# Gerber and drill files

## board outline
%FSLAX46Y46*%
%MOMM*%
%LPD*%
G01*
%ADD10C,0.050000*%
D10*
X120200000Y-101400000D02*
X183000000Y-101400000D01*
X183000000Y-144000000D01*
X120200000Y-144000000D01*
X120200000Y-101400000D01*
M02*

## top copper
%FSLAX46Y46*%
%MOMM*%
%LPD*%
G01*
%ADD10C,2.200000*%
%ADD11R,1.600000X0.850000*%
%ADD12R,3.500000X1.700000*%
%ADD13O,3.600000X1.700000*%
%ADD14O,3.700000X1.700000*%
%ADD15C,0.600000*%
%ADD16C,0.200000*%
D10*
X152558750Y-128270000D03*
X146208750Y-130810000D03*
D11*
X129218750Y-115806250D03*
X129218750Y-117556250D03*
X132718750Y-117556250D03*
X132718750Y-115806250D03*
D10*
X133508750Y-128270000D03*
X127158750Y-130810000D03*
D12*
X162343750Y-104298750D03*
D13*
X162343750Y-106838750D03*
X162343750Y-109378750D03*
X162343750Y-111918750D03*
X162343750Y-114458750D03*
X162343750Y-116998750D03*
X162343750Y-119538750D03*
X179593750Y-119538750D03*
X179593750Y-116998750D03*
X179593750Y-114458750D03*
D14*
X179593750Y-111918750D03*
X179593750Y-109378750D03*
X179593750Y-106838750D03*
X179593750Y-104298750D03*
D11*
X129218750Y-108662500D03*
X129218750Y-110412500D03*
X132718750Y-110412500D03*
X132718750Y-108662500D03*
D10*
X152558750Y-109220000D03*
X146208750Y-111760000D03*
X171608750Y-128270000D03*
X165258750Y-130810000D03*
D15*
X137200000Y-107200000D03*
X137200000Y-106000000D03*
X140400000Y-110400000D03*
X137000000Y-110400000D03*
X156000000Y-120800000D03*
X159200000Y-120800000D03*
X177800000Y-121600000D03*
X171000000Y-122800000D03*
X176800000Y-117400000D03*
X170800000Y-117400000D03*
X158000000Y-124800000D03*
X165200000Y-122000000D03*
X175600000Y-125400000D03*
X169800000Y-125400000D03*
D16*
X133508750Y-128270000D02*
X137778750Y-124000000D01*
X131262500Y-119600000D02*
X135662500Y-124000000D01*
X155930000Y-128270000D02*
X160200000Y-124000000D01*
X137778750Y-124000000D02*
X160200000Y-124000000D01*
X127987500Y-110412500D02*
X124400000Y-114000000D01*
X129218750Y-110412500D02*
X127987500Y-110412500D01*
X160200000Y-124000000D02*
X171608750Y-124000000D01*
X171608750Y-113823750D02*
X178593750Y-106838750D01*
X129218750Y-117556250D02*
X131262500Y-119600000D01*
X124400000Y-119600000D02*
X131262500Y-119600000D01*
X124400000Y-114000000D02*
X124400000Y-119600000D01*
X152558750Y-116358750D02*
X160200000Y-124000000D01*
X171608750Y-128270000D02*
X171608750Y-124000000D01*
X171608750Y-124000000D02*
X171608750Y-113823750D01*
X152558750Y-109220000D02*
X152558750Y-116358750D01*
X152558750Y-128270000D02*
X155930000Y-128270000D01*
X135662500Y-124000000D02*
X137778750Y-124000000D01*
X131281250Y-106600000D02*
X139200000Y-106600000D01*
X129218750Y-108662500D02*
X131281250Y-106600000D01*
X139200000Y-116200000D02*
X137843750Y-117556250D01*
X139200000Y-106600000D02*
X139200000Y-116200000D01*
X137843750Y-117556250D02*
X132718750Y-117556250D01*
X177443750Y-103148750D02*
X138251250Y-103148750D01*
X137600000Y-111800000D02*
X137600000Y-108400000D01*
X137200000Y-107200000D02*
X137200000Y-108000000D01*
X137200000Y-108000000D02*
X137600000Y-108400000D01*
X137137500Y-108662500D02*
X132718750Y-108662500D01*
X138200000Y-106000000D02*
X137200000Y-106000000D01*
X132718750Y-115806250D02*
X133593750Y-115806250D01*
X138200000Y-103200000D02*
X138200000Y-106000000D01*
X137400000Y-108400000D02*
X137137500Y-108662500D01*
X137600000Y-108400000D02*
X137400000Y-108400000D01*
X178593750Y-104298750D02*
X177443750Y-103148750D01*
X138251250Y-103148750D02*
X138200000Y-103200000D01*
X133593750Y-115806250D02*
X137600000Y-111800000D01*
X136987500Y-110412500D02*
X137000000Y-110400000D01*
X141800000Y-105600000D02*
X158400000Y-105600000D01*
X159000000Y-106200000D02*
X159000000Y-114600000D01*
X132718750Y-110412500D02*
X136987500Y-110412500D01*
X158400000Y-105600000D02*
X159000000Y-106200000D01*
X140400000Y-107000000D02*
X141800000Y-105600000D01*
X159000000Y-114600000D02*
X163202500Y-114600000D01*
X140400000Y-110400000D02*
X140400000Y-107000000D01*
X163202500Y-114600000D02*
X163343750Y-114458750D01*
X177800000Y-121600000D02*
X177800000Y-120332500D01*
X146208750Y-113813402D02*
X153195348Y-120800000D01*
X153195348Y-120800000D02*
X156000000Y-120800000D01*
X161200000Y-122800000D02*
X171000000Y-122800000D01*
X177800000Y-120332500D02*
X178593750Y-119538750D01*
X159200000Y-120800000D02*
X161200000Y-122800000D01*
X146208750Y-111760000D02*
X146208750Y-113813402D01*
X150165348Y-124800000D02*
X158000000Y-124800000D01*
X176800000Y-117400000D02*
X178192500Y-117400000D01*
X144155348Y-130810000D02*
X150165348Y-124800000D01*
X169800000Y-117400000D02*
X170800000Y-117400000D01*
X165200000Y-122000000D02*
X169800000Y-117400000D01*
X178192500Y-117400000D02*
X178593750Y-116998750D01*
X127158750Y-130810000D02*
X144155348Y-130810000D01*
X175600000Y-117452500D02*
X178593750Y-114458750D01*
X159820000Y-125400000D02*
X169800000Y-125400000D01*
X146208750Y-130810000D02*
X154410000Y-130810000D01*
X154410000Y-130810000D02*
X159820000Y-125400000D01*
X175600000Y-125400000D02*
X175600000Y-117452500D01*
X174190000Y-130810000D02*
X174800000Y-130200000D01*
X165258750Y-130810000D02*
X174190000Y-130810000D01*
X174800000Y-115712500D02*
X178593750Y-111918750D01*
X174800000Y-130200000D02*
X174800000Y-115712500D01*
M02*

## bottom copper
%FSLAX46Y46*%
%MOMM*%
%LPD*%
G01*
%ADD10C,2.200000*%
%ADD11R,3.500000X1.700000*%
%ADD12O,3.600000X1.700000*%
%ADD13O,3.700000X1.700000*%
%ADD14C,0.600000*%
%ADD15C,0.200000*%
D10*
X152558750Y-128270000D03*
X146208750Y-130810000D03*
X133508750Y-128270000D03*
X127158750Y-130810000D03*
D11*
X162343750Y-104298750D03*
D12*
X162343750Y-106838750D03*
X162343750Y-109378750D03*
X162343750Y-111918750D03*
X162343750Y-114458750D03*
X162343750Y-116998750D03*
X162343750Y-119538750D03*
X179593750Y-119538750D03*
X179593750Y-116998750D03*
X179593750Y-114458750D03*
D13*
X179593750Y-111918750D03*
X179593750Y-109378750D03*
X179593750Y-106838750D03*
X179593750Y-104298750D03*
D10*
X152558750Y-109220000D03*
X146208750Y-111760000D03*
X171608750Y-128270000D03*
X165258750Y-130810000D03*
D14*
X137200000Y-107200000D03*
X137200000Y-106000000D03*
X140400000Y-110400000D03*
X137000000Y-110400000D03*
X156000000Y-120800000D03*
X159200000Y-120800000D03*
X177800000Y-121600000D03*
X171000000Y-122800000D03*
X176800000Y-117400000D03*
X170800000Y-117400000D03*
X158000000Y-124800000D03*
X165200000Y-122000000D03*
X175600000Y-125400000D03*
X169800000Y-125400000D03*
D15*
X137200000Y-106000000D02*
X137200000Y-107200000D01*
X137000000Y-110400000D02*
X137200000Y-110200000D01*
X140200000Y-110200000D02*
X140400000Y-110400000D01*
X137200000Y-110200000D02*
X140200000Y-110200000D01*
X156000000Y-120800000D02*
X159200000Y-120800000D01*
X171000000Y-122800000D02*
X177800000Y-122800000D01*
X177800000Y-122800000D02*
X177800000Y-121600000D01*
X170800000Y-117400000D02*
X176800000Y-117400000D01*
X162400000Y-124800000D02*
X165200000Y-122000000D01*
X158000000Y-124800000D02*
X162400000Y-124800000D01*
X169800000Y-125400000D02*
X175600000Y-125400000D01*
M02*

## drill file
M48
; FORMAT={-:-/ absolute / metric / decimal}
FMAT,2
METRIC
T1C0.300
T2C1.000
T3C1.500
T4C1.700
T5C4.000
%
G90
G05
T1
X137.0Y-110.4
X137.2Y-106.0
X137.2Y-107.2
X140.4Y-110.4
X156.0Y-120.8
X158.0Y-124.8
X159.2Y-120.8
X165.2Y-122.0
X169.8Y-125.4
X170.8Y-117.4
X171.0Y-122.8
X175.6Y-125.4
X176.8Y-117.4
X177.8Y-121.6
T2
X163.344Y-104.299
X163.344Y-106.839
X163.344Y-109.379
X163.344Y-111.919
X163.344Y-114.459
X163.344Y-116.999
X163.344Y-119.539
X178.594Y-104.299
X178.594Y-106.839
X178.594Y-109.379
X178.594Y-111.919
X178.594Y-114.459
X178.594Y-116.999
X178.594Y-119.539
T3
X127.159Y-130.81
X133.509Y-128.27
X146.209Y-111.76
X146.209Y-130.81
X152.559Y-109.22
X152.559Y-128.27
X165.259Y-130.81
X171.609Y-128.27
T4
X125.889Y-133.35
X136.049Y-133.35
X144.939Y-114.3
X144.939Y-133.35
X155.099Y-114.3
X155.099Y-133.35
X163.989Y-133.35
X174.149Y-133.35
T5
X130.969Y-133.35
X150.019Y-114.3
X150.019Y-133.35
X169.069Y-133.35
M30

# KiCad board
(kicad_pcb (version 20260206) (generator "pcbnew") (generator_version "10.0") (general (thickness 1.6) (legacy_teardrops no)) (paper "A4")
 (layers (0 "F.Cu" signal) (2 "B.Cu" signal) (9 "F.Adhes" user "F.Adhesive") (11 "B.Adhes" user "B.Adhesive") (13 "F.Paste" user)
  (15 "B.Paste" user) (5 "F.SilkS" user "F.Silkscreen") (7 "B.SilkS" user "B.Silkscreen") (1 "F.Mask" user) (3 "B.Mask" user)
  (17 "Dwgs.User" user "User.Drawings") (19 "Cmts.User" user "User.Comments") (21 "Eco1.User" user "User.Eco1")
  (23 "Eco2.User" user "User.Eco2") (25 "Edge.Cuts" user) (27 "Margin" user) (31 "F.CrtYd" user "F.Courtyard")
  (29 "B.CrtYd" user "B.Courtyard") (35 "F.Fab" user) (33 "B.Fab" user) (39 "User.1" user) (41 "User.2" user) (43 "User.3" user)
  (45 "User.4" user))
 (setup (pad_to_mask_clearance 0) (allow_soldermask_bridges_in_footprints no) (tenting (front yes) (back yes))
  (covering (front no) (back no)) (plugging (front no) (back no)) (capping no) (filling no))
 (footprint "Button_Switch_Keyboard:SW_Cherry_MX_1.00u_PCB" (layer "F.Cu") (at 152.55875 128.27)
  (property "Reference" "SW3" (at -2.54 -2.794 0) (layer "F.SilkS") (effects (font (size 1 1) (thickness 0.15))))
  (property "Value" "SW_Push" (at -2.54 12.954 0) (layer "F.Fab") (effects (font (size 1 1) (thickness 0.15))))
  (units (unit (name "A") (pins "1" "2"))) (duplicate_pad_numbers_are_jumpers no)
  (pad "" np_thru_hole circle (at -7.62 5.08) (size 1.7 1.7) (drill 1.7) (layers "*.Cu" "*.Mask"))
  (pad "" np_thru_hole circle (at -2.54 5.08) (size 4 4) (drill 4) (layers "*.Cu" "*.Mask"))
  (pad "" np_thru_hole circle (at 2.54 5.08) (size 1.7 1.7) (drill 1.7) (layers "*.Cu" "*.Mask"))
  (pad "1" thru_hole circle (at 0 0) (size 2.2 2.2) (drill 1.5) (layers "*.Cu" "*.Mask") (remove_unused_layers no) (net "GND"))
  (pad "2" thru_hole circle (at -6.35 2.54) (size 2.2 2.2) (drill 1.5) (layers "*.Cu" "*.Mask") (remove_unused_layers no)
   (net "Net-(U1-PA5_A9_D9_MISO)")))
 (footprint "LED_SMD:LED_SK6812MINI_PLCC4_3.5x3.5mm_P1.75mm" (layer "F.Cu") (at 130.96875 116.68125)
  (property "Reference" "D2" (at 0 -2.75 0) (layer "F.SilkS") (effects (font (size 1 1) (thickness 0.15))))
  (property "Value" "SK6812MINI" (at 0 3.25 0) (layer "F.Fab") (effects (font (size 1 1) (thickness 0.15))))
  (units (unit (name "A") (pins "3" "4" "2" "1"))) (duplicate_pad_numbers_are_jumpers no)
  (pad "1" smd rect (at -1.75 -0.875) (size 1.6 0.85) (layers "F.Cu" "F.Mask" "F.Paste") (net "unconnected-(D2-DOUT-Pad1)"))
  (pad "2" smd rect (at -1.75 0.875) (size 1.6 0.85) (layers "F.Cu" "F.Mask" "F.Paste") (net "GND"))
  (pad "3" smd rect (at 1.75 0.875) (size 1.6 0.85) (layers "F.Cu" "F.Mask" "F.Paste") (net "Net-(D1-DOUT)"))
  (pad "4" smd rect (at 1.75 -0.875) (size 1.6 0.85) (layers "F.Cu" "F.Mask" "F.Paste") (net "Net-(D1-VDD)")))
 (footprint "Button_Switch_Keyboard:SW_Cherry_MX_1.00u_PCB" (layer "F.Cu") (at 133.50875 128.27)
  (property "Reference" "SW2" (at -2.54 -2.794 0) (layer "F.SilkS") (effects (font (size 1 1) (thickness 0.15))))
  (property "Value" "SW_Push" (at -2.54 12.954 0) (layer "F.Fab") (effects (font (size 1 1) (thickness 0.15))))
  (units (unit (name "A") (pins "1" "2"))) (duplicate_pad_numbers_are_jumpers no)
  (pad "" np_thru_hole circle (at -7.62 5.08) (size 1.7 1.7) (drill 1.7) (layers "*.Cu" "*.Mask"))
  (pad "" np_thru_hole circle (at -2.54 5.08) (size 4 4) (drill 4) (layers "*.Cu" "*.Mask"))
  (pad "" np_thru_hole circle (at 2.54 5.08) (size 1.7 1.7) (drill 1.7) (layers "*.Cu" "*.Mask"))
  (pad "1" thru_hole circle (at 0 0) (size 2.2 2.2) (drill 1.5) (layers "*.Cu" "*.Mask") (remove_unused_layers no) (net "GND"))
  (pad "2" thru_hole circle (at -6.35 2.54) (size 2.2 2.2) (drill 1.5) (layers "*.Cu" "*.Mask") (remove_unused_layers no)
   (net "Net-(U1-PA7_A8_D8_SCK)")))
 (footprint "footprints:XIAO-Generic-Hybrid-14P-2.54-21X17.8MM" (layer "F.Cu") (at 170.96875 111.91875)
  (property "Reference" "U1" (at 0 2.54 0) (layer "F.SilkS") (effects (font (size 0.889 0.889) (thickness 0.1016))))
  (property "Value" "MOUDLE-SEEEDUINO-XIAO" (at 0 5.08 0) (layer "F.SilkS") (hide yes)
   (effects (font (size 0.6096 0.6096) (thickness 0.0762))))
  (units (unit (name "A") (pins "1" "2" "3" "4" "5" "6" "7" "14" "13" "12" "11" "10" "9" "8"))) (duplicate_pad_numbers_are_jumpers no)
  (pad "1" thru_hole rect (at -7.625 -7.62) (size 3.5 1.7) (drill 1 (offset -1 0)) (layers "*.Cu" "*.Mask") (remove_unused_layers no)
   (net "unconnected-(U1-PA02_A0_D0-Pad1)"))
  (pad "2" thru_hole oval (at -7.625 -5.08) (size 3.6 1.7) (drill 1 (offset -1 0)) (layers "*.Cu" "*.Mask") (remove_unused_layers no)
   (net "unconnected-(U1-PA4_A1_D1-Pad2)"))
  (pad "3" thru_hole oval (at -7.625 -2.54) (size 3.6 1.7) (drill 1 (offset -1 0)) (layers "*.Cu" "*.Mask") (remove_unused_layers no)
   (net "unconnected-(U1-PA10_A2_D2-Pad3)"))
  (pad "4" thru_hole oval (at -7.625 0) (size 3.6 1.7) (drill 1 (offset -1 0)) (layers "*.Cu" "*.Mask") (remove_unused_layers no)
   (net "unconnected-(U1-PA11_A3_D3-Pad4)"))
  (pad "5" thru_hole oval (at -7.625 2.54) (size 3.6 1.7) (drill 1 (offset -1 0)) (layers "*.Cu" "*.Mask") (remove_unused_layers no)
   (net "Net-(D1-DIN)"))
  (pad "6" thru_hole oval (at -7.625 5.08 180) (size 3.6 1.7) (drill 1 (offset 1 0)) (layers "*.Cu" "*.Mask") (remove_unused_layers no)
   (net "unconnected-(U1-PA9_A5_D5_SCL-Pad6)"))
  (pad "7" thru_hole oval (at -7.625 7.62) (size 3.6 1.7) (drill 1 (offset -1 0)) (layers "*.Cu" "*.Mask") (remove_unused_layers no)
   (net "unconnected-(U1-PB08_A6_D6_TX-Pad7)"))
  (pad "8" thru_hole oval (at 7.625 7.62) (size 3.6 1.7) (drill 1 (offset 1 0)) (layers "*.Cu" "*.Mask") (remove_unused_layers no)
   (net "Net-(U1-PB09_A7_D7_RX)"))
  (pad "9" thru_hole oval (at 7.625 5.08) (size 3.6 1.7) (drill 1 (offset 1 0)) (layers "*.Cu" "*.Mask") (remove_unused_layers no)
   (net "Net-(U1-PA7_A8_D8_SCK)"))
  (pad "10" thru_hole oval (at 7.625 2.54) (size 3.6 1.7) (drill 1 (offset 1 0)) (layers "*.Cu" "*.Mask") (remove_unused_layers no)
   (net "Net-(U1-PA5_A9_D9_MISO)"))
  (pad "11" thru_hole oval (at 7.625 0) (size 3.7 1.7) (drill 1 (offset 1 0)) (layers "*.Cu" "*.Mask") (remove_unused_layers no)
   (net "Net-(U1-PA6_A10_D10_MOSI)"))
  (pad "12" thru_hole oval (at 7.625 -2.54) (size 3.7 1.7) (drill 1 (offset 1 0)) (layers "*.Cu" "*.Mask") (remove_unused_layers no)
   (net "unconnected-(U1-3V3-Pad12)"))
  (pad "13" thru_hole oval (at 7.625 -5.08) (size 3.7 1.7) (drill 1 (offset 1 0)) (layers "*.Cu" "*.Mask") (remove_unused_layers no)
   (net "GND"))
  (pad "14" thru_hole oval (at 7.625 -7.62) (size 3.7 1.7) (drill 1 (offset 1 0)) (layers "*.Cu" "*.Mask") (remove_unused_layers no)
   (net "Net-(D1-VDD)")))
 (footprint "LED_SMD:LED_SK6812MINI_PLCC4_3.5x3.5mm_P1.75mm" (layer "F.Cu") (at 130.96875 109.5375)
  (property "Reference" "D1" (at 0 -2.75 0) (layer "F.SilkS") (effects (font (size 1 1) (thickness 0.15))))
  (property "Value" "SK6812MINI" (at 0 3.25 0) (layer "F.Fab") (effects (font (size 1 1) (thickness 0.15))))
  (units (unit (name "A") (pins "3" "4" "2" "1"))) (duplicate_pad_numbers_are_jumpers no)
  (pad "1" smd rect (at -1.75 -0.875) (size 1.6 0.85) (layers "F.Cu" "F.Mask" "F.Paste") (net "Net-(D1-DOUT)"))
  (pad "2" smd rect (at -1.75 0.875) (size 1.6 0.85) (layers "F.Cu" "F.Mask" "F.Paste") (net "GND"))
  (pad "3" smd rect (at 1.75 0.875) (size 1.6 0.85) (layers "F.Cu" "F.Mask" "F.Paste") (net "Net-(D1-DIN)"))
  (pad "4" smd rect (at 1.75 -0.875) (size 1.6 0.85) (layers "F.Cu" "F.Mask" "F.Paste") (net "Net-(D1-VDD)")))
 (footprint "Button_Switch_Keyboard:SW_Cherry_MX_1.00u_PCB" (layer "F.Cu") (at 152.55875 109.22)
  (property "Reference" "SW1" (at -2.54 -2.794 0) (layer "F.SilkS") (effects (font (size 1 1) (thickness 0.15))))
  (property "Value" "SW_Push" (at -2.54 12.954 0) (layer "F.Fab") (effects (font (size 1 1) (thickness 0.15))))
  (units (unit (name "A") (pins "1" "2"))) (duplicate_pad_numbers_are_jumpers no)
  (pad "" np_thru_hole circle (at -7.62 5.08) (size 1.7 1.7) (drill 1.7) (layers "*.Cu" "*.Mask"))
  (pad "" np_thru_hole circle (at -2.54 5.08) (size 4 4) (drill 4) (layers "*.Cu" "*.Mask"))
  (pad "" np_thru_hole circle (at 2.54 5.08) (size 1.7 1.7) (drill 1.7) (layers "*.Cu" "*.Mask"))
  (pad "1" thru_hole circle (at 0 0) (size 2.2 2.2) (drill 1.5) (layers "*.Cu" "*.Mask") (remove_unused_layers no) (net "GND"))
  (pad "2" thru_hole circle (at -6.35 2.54) (size 2.2 2.2) (drill 1.5) (layers "*.Cu" "*.Mask") (remove_unused_layers no)
   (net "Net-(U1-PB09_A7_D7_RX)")))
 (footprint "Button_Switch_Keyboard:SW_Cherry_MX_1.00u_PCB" (layer "F.Cu") (at 171.60875 128.27)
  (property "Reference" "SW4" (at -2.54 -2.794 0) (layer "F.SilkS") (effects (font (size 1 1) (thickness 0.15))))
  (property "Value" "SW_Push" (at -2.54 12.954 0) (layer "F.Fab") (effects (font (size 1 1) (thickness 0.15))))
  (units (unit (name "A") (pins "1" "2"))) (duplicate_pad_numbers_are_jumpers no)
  (pad "" np_thru_hole circle (at -7.62 5.08) (size 1.7 1.7) (drill 1.7) (layers "*.Cu" "*.Mask"))
  (pad "" np_thru_hole circle (at -2.54 5.08) (size 4 4) (drill 4) (layers "*.Cu" "*.Mask"))
  (pad "" np_thru_hole circle (at 2.54 5.08) (size 1.7 1.7) (drill 1.7) (layers "*.Cu" "*.Mask"))
  (pad "1" thru_hole circle (at 0 0) (size 2.2 2.2) (drill 1.5) (layers "*.Cu" "*.Mask") (remove_unused_layers no) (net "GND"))
  (pad "2" thru_hole circle (at -6.35 2.54) (size 2.2 2.2) (drill 1.5) (layers "*.Cu" "*.Mask") (remove_unused_layers no)
   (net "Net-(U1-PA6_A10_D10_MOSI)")))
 (gr_rect (start 120.2 101.4) (end 183 144) (stroke (width 0.05) (type default)) (fill no) (layer "Edge.Cuts"))
 (segment (start 133.50875 128.27) (end 137.77875 124) (width 0.2) (layer "F.Cu") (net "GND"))
 (segment (start 131.2625 119.6) (end 135.6625 124) (width 0.2) (layer "F.Cu") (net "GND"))
 (segment (start 155.93 128.27) (end 160.2 124) (width 0.2) (layer "F.Cu") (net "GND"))
 (segment (start 137.77875 124) (end 160.2 124) (width 0.2) (layer "F.Cu") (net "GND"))
 (segment (start 127.9875 110.4125) (end 124.4 114) (width 0.2) (layer "F.Cu") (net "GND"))
 (segment (start 129.21875 110.4125) (end 127.9875 110.4125) (width 0.2) (layer "F.Cu") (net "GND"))
 (segment (start 160.2 124) (end 171.60875 124) (width 0.2) (layer "F.Cu") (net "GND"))
 (segment (start 171.60875 113.82375) (end 178.59375 106.83875) (width 0.2) (layer "F.Cu") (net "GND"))
 (segment (start 129.21875 117.55625) (end 131.2625 119.6) (width 0.2) (layer "F.Cu") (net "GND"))
 (segment (start 124.4 119.6) (end 131.2625 119.6) (width 0.2) (layer "F.Cu") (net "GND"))
 (segment (start 124.4 114) (end 124.4 119.6) (width 0.2) (layer "F.Cu") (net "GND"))
 (segment (start 152.55875 116.35875) (end 160.2 124) (width 0.2) (layer "F.Cu") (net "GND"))
 (segment (start 171.60875 128.27) (end 171.60875 124) (width 0.2) (layer "F.Cu") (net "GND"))
 (segment (start 171.60875 124) (end 171.60875 113.82375) (width 0.2) (layer "F.Cu") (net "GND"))
 (segment (start 152.55875 109.22) (end 152.55875 116.35875) (width 0.2) (layer "F.Cu") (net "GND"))
 (segment (start 152.55875 128.27) (end 155.93 128.27) (width 0.2) (layer "F.Cu") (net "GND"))
 (segment (start 135.6625 124) (end 137.77875 124) (width 0.2) (layer "F.Cu") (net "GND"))
 (segment (start 131.28125 106.6) (end 139.2 106.6) (width 0.2) (layer "F.Cu") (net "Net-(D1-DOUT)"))
 (segment (start 129.21875 108.6625) (end 131.28125 106.6) (width 0.2) (layer "F.Cu") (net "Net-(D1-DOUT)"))
 (segment (start 139.2 116.2) (end 137.84375 117.55625) (width 0.2) (layer "F.Cu") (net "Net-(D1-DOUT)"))
 (segment (start 139.2 106.6) (end 139.2 116.2) (width 0.2) (layer "F.Cu") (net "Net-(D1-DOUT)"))
 (segment (start 137.84375 117.55625) (end 132.71875 117.55625) (width 0.2) (layer "F.Cu") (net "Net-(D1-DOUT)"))
 (segment (start 177.44375 103.14875) (end 138.25125 103.14875) (width 0.2) (layer "F.Cu") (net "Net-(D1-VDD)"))
 (segment (start 137.6 111.8) (end 137.6 108.4) (width 0.2) (layer "F.Cu") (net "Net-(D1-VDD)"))
 (segment (start 137.2 107.2) (end 137.2 108) (width 0.2) (layer "F.Cu") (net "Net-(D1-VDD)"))
 (segment (start 137.2 108) (end 137.6 108.4) (width 0.2) (layer "F.Cu") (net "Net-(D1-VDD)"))
 (segment (start 137.1375 108.6625) (end 132.71875 108.6625) (width 0.2) (layer "F.Cu") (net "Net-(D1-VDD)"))
 (segment (start 138.2 106) (end 137.2 106) (width 0.2) (layer "F.Cu") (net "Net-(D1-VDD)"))
 (segment (start 132.71875 115.80625) (end 133.59375 115.80625) (width 0.2) (layer "F.Cu") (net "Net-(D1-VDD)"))
 (segment (start 138.2 103.2) (end 138.2 106) (width 0.2) (layer "F.Cu") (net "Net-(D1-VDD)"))
 (segment (start 137.4 108.4) (end 137.1375 108.6625) (width 0.2) (layer "F.Cu") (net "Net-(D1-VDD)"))
 (segment (start 137.6 108.4) (end 137.4 108.4) (width 0.2) (layer "F.Cu") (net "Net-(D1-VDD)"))
 (segment (start 178.59375 104.29875) (end 177.44375 103.14875) (width 0.2) (layer "F.Cu") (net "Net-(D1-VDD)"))
 (segment (start 138.25125 103.14875) (end 138.2 103.2) (width 0.2) (layer "F.Cu") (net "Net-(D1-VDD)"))
 (segment (start 133.59375 115.80625) (end 137.6 111.8) (width 0.2) (layer "F.Cu") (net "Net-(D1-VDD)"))
 (via (at 137.2 107.2) (size 0.6) (drill 0.3) (layers "F.Cu" "B.Cu") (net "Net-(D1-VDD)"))
 (via (at 137.2 106) (size 0.6) (drill 0.3) (layers "F.Cu" "B.Cu") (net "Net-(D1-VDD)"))
 (segment (start 137.2 106) (end 137.2 107.2) (width 0.2) (layer "B.Cu") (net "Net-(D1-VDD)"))
 (segment (start 136.9875 110.4125) (end 137 110.4) (width 0.2) (layer "F.Cu") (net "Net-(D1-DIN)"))
 (segment (start 141.8 105.6) (end 158.4 105.6) (width 0.2) (layer "F.Cu") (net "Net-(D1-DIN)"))
 (segment (start 159 106.2) (end 159 114.6) (width 0.2) (layer "F.Cu") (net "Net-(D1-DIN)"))
 (segment (start 132.71875 110.4125) (end 136.9875 110.4125) (width 0.2) (layer "F.Cu") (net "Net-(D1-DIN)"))
 (segment (start 158.4 105.6) (end 159 106.2) (width 0.2) (layer "F.Cu") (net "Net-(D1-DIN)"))
 (segment (start 140.4 107) (end 141.8 105.6) (width 0.2) (layer "F.Cu") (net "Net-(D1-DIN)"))
 (segment (start 159 114.6) (end 163.2025 114.6) (width 0.2) (layer "F.Cu") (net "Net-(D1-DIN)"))
 (segment (start 140.4 110.4) (end 140.4 107) (width 0.2) (layer "F.Cu") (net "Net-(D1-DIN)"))
 (segment (start 163.2025 114.6) (end 163.34375 114.45875) (width 0.2) (layer "F.Cu") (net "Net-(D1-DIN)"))
 (via (at 140.4 110.4) (size 0.6) (drill 0.3) (layers "F.Cu" "B.Cu") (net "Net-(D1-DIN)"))
 (via (at 137 110.4) (size 0.6) (drill 0.3) (layers "F.Cu" "B.Cu") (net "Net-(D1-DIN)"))
 (segment (start 137 110.4) (end 137.2 110.2) (width 0.2) (layer "B.Cu") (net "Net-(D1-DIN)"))
 (segment (start 140.2 110.2) (end 140.4 110.4) (width 0.2) (layer "B.Cu") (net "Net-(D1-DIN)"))
 (segment (start 137.2 110.2) (end 140.2 110.2) (width 0.2) (layer "B.Cu") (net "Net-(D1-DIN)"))
 (segment (start 177.8 121.6) (end 177.8 120.3325) (width 0.2) (layer "F.Cu") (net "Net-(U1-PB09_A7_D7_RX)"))
 (segment (start 146.20875 113.813402) (end 153.195348 120.8) (width 0.2) (layer "F.Cu") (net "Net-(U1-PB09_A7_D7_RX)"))
 (segment (start 153.195348 120.8) (end 156 120.8) (width 0.2) (layer "F.Cu") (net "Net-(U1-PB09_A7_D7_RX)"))
 (segment (start 161.2 122.8) (end 171 122.8) (width 0.2) (layer "F.Cu") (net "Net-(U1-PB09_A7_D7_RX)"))
 (segment (start 177.8 120.3325) (end 178.59375 119.53875) (width 0.2) (layer "F.Cu") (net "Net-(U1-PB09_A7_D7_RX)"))
 (segment (start 159.2 120.8) (end 161.2 122.8) (width 0.2) (layer "F.Cu") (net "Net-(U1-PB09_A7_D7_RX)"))
 (segment (start 146.20875 111.76) (end 146.20875 113.813402) (width 0.2) (layer "F.Cu") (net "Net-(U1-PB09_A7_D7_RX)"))
 (via (at 156 120.8) (size 0.6) (drill 0.3) (layers "F.Cu" "B.Cu") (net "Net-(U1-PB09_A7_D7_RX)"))
 (via (at 159.2 120.8) (size 0.6) (drill 0.3) (layers "F.Cu" "B.Cu") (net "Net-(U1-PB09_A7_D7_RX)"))
 (via (at 177.8 121.6) (size 0.6) (drill 0.3) (layers "F.Cu" "B.Cu") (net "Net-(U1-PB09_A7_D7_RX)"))
 (via (at 171 122.8) (size 0.6) (drill 0.3) (layers "F.Cu" "B.Cu") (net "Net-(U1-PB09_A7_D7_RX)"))
 (segment (start 156 120.8) (end 159.2 120.8) (width 0.2) (layer "B.Cu") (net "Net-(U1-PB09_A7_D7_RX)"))
 (segment (start 171 122.8) (end 177.8 122.8) (width 0.2) (layer "B.Cu") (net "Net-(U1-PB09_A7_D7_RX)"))
 (segment (start 177.8 122.8) (end 177.8 121.6) (width 0.2) (layer "B.Cu") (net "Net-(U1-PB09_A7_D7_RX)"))
 (segment (start 150.165348 124.8) (end 158 124.8) (width 0.2) (layer "F.Cu") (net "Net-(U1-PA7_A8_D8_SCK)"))
 (segment (start 176.8 117.4) (end 178.1925 117.4) (width 0.2) (layer "F.Cu") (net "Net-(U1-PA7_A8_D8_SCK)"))
 (segment (start 144.155348 130.81) (end 150.165348 124.8) (width 0.2) (layer "F.Cu") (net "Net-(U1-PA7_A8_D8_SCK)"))
 (segment (start 169.8 117.4) (end 170.8 117.4) (width 0.2) (layer "F.Cu") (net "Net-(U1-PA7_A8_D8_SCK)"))
 (segment (start 165.2 122) (end 169.8 117.4) (width 0.2) (layer "F.Cu") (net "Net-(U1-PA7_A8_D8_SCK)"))
 (segment (start 178.1925 117.4) (end 178.59375 116.99875) (width 0.2) (layer "F.Cu") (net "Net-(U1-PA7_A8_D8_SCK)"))
 (segment (start 127.15875 130.81) (end 144.155348 130.81) (width 0.2) (layer "F.Cu") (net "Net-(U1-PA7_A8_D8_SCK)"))
 (via (at 176.8 117.4) (size 0.6) (drill 0.3) (layers "F.Cu" "B.Cu") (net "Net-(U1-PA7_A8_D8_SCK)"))
 (via (at 170.8 117.4) (size 0.6) (drill 0.3) (layers "F.Cu" "B.Cu") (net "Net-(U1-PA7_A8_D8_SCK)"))
 (via (at 158 124.8) (size 0.6) (drill 0.3) (layers "F.Cu" "B.Cu") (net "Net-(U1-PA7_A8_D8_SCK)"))
 (via (at 165.2 122) (size 0.6) (drill 0.3) (layers "F.Cu" "B.Cu") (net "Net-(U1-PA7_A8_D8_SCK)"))
 (segment (start 170.8 117.4) (end 176.8 117.4) (width 0.2) (layer "B.Cu") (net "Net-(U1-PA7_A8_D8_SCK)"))
 (segment (start 162.4 124.8) (end 165.2 122) (width 0.2) (layer "B.Cu") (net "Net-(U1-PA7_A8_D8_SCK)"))
 (segment (start 158 124.8) (end 162.4 124.8) (width 0.2) (layer "B.Cu") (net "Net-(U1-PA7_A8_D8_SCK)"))
 (segment (start 175.6 117.4525) (end 178.59375 114.45875) (width 0.2) (layer "F.Cu") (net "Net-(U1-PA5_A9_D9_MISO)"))
 (segment (start 159.82 125.4) (end 169.8 125.4) (width 0.2) (layer "F.Cu") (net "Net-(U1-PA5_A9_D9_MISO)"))
 (segment (start 146.20875 130.81) (end 154.41 130.81) (width 0.2) (layer "F.Cu") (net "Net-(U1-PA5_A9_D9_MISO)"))
 (segment (start 154.41 130.81) (end 159.82 125.4) (width 0.2) (layer "F.Cu") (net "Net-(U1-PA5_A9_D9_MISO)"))
 (segment (start 175.6 125.4) (end 175.6 117.4525) (width 0.2) (layer "F.Cu") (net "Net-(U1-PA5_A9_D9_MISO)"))
 (via (at 175.6 125.4) (size 0.6) (drill 0.3) (layers "F.Cu" "B.Cu") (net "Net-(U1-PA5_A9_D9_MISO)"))
 (via (at 169.8 125.4) (size 0.6) (drill 0.3) (layers "F.Cu" "B.Cu") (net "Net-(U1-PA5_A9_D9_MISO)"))
 (segment (start 169.8 125.4) (end 175.6 125.4) (width 0.2) (layer "B.Cu") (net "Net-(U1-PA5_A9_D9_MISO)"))
 (segment (start 174.19 130.81) (end 174.8 130.2) (width 0.2) (layer "F.Cu") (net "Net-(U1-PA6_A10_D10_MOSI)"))
 (segment (start 165.25875 130.81) (end 174.19 130.81) (width 0.2) (layer "F.Cu") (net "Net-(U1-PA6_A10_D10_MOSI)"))
 (segment (start 174.8 115.7125) (end 178.59375 111.91875) (width 0.2) (layer "F.Cu") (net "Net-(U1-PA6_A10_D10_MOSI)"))
 (segment (start 174.8 130.2) (end 174.8 115.7125) (width 0.2) (layer "F.Cu") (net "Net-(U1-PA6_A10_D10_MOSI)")))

